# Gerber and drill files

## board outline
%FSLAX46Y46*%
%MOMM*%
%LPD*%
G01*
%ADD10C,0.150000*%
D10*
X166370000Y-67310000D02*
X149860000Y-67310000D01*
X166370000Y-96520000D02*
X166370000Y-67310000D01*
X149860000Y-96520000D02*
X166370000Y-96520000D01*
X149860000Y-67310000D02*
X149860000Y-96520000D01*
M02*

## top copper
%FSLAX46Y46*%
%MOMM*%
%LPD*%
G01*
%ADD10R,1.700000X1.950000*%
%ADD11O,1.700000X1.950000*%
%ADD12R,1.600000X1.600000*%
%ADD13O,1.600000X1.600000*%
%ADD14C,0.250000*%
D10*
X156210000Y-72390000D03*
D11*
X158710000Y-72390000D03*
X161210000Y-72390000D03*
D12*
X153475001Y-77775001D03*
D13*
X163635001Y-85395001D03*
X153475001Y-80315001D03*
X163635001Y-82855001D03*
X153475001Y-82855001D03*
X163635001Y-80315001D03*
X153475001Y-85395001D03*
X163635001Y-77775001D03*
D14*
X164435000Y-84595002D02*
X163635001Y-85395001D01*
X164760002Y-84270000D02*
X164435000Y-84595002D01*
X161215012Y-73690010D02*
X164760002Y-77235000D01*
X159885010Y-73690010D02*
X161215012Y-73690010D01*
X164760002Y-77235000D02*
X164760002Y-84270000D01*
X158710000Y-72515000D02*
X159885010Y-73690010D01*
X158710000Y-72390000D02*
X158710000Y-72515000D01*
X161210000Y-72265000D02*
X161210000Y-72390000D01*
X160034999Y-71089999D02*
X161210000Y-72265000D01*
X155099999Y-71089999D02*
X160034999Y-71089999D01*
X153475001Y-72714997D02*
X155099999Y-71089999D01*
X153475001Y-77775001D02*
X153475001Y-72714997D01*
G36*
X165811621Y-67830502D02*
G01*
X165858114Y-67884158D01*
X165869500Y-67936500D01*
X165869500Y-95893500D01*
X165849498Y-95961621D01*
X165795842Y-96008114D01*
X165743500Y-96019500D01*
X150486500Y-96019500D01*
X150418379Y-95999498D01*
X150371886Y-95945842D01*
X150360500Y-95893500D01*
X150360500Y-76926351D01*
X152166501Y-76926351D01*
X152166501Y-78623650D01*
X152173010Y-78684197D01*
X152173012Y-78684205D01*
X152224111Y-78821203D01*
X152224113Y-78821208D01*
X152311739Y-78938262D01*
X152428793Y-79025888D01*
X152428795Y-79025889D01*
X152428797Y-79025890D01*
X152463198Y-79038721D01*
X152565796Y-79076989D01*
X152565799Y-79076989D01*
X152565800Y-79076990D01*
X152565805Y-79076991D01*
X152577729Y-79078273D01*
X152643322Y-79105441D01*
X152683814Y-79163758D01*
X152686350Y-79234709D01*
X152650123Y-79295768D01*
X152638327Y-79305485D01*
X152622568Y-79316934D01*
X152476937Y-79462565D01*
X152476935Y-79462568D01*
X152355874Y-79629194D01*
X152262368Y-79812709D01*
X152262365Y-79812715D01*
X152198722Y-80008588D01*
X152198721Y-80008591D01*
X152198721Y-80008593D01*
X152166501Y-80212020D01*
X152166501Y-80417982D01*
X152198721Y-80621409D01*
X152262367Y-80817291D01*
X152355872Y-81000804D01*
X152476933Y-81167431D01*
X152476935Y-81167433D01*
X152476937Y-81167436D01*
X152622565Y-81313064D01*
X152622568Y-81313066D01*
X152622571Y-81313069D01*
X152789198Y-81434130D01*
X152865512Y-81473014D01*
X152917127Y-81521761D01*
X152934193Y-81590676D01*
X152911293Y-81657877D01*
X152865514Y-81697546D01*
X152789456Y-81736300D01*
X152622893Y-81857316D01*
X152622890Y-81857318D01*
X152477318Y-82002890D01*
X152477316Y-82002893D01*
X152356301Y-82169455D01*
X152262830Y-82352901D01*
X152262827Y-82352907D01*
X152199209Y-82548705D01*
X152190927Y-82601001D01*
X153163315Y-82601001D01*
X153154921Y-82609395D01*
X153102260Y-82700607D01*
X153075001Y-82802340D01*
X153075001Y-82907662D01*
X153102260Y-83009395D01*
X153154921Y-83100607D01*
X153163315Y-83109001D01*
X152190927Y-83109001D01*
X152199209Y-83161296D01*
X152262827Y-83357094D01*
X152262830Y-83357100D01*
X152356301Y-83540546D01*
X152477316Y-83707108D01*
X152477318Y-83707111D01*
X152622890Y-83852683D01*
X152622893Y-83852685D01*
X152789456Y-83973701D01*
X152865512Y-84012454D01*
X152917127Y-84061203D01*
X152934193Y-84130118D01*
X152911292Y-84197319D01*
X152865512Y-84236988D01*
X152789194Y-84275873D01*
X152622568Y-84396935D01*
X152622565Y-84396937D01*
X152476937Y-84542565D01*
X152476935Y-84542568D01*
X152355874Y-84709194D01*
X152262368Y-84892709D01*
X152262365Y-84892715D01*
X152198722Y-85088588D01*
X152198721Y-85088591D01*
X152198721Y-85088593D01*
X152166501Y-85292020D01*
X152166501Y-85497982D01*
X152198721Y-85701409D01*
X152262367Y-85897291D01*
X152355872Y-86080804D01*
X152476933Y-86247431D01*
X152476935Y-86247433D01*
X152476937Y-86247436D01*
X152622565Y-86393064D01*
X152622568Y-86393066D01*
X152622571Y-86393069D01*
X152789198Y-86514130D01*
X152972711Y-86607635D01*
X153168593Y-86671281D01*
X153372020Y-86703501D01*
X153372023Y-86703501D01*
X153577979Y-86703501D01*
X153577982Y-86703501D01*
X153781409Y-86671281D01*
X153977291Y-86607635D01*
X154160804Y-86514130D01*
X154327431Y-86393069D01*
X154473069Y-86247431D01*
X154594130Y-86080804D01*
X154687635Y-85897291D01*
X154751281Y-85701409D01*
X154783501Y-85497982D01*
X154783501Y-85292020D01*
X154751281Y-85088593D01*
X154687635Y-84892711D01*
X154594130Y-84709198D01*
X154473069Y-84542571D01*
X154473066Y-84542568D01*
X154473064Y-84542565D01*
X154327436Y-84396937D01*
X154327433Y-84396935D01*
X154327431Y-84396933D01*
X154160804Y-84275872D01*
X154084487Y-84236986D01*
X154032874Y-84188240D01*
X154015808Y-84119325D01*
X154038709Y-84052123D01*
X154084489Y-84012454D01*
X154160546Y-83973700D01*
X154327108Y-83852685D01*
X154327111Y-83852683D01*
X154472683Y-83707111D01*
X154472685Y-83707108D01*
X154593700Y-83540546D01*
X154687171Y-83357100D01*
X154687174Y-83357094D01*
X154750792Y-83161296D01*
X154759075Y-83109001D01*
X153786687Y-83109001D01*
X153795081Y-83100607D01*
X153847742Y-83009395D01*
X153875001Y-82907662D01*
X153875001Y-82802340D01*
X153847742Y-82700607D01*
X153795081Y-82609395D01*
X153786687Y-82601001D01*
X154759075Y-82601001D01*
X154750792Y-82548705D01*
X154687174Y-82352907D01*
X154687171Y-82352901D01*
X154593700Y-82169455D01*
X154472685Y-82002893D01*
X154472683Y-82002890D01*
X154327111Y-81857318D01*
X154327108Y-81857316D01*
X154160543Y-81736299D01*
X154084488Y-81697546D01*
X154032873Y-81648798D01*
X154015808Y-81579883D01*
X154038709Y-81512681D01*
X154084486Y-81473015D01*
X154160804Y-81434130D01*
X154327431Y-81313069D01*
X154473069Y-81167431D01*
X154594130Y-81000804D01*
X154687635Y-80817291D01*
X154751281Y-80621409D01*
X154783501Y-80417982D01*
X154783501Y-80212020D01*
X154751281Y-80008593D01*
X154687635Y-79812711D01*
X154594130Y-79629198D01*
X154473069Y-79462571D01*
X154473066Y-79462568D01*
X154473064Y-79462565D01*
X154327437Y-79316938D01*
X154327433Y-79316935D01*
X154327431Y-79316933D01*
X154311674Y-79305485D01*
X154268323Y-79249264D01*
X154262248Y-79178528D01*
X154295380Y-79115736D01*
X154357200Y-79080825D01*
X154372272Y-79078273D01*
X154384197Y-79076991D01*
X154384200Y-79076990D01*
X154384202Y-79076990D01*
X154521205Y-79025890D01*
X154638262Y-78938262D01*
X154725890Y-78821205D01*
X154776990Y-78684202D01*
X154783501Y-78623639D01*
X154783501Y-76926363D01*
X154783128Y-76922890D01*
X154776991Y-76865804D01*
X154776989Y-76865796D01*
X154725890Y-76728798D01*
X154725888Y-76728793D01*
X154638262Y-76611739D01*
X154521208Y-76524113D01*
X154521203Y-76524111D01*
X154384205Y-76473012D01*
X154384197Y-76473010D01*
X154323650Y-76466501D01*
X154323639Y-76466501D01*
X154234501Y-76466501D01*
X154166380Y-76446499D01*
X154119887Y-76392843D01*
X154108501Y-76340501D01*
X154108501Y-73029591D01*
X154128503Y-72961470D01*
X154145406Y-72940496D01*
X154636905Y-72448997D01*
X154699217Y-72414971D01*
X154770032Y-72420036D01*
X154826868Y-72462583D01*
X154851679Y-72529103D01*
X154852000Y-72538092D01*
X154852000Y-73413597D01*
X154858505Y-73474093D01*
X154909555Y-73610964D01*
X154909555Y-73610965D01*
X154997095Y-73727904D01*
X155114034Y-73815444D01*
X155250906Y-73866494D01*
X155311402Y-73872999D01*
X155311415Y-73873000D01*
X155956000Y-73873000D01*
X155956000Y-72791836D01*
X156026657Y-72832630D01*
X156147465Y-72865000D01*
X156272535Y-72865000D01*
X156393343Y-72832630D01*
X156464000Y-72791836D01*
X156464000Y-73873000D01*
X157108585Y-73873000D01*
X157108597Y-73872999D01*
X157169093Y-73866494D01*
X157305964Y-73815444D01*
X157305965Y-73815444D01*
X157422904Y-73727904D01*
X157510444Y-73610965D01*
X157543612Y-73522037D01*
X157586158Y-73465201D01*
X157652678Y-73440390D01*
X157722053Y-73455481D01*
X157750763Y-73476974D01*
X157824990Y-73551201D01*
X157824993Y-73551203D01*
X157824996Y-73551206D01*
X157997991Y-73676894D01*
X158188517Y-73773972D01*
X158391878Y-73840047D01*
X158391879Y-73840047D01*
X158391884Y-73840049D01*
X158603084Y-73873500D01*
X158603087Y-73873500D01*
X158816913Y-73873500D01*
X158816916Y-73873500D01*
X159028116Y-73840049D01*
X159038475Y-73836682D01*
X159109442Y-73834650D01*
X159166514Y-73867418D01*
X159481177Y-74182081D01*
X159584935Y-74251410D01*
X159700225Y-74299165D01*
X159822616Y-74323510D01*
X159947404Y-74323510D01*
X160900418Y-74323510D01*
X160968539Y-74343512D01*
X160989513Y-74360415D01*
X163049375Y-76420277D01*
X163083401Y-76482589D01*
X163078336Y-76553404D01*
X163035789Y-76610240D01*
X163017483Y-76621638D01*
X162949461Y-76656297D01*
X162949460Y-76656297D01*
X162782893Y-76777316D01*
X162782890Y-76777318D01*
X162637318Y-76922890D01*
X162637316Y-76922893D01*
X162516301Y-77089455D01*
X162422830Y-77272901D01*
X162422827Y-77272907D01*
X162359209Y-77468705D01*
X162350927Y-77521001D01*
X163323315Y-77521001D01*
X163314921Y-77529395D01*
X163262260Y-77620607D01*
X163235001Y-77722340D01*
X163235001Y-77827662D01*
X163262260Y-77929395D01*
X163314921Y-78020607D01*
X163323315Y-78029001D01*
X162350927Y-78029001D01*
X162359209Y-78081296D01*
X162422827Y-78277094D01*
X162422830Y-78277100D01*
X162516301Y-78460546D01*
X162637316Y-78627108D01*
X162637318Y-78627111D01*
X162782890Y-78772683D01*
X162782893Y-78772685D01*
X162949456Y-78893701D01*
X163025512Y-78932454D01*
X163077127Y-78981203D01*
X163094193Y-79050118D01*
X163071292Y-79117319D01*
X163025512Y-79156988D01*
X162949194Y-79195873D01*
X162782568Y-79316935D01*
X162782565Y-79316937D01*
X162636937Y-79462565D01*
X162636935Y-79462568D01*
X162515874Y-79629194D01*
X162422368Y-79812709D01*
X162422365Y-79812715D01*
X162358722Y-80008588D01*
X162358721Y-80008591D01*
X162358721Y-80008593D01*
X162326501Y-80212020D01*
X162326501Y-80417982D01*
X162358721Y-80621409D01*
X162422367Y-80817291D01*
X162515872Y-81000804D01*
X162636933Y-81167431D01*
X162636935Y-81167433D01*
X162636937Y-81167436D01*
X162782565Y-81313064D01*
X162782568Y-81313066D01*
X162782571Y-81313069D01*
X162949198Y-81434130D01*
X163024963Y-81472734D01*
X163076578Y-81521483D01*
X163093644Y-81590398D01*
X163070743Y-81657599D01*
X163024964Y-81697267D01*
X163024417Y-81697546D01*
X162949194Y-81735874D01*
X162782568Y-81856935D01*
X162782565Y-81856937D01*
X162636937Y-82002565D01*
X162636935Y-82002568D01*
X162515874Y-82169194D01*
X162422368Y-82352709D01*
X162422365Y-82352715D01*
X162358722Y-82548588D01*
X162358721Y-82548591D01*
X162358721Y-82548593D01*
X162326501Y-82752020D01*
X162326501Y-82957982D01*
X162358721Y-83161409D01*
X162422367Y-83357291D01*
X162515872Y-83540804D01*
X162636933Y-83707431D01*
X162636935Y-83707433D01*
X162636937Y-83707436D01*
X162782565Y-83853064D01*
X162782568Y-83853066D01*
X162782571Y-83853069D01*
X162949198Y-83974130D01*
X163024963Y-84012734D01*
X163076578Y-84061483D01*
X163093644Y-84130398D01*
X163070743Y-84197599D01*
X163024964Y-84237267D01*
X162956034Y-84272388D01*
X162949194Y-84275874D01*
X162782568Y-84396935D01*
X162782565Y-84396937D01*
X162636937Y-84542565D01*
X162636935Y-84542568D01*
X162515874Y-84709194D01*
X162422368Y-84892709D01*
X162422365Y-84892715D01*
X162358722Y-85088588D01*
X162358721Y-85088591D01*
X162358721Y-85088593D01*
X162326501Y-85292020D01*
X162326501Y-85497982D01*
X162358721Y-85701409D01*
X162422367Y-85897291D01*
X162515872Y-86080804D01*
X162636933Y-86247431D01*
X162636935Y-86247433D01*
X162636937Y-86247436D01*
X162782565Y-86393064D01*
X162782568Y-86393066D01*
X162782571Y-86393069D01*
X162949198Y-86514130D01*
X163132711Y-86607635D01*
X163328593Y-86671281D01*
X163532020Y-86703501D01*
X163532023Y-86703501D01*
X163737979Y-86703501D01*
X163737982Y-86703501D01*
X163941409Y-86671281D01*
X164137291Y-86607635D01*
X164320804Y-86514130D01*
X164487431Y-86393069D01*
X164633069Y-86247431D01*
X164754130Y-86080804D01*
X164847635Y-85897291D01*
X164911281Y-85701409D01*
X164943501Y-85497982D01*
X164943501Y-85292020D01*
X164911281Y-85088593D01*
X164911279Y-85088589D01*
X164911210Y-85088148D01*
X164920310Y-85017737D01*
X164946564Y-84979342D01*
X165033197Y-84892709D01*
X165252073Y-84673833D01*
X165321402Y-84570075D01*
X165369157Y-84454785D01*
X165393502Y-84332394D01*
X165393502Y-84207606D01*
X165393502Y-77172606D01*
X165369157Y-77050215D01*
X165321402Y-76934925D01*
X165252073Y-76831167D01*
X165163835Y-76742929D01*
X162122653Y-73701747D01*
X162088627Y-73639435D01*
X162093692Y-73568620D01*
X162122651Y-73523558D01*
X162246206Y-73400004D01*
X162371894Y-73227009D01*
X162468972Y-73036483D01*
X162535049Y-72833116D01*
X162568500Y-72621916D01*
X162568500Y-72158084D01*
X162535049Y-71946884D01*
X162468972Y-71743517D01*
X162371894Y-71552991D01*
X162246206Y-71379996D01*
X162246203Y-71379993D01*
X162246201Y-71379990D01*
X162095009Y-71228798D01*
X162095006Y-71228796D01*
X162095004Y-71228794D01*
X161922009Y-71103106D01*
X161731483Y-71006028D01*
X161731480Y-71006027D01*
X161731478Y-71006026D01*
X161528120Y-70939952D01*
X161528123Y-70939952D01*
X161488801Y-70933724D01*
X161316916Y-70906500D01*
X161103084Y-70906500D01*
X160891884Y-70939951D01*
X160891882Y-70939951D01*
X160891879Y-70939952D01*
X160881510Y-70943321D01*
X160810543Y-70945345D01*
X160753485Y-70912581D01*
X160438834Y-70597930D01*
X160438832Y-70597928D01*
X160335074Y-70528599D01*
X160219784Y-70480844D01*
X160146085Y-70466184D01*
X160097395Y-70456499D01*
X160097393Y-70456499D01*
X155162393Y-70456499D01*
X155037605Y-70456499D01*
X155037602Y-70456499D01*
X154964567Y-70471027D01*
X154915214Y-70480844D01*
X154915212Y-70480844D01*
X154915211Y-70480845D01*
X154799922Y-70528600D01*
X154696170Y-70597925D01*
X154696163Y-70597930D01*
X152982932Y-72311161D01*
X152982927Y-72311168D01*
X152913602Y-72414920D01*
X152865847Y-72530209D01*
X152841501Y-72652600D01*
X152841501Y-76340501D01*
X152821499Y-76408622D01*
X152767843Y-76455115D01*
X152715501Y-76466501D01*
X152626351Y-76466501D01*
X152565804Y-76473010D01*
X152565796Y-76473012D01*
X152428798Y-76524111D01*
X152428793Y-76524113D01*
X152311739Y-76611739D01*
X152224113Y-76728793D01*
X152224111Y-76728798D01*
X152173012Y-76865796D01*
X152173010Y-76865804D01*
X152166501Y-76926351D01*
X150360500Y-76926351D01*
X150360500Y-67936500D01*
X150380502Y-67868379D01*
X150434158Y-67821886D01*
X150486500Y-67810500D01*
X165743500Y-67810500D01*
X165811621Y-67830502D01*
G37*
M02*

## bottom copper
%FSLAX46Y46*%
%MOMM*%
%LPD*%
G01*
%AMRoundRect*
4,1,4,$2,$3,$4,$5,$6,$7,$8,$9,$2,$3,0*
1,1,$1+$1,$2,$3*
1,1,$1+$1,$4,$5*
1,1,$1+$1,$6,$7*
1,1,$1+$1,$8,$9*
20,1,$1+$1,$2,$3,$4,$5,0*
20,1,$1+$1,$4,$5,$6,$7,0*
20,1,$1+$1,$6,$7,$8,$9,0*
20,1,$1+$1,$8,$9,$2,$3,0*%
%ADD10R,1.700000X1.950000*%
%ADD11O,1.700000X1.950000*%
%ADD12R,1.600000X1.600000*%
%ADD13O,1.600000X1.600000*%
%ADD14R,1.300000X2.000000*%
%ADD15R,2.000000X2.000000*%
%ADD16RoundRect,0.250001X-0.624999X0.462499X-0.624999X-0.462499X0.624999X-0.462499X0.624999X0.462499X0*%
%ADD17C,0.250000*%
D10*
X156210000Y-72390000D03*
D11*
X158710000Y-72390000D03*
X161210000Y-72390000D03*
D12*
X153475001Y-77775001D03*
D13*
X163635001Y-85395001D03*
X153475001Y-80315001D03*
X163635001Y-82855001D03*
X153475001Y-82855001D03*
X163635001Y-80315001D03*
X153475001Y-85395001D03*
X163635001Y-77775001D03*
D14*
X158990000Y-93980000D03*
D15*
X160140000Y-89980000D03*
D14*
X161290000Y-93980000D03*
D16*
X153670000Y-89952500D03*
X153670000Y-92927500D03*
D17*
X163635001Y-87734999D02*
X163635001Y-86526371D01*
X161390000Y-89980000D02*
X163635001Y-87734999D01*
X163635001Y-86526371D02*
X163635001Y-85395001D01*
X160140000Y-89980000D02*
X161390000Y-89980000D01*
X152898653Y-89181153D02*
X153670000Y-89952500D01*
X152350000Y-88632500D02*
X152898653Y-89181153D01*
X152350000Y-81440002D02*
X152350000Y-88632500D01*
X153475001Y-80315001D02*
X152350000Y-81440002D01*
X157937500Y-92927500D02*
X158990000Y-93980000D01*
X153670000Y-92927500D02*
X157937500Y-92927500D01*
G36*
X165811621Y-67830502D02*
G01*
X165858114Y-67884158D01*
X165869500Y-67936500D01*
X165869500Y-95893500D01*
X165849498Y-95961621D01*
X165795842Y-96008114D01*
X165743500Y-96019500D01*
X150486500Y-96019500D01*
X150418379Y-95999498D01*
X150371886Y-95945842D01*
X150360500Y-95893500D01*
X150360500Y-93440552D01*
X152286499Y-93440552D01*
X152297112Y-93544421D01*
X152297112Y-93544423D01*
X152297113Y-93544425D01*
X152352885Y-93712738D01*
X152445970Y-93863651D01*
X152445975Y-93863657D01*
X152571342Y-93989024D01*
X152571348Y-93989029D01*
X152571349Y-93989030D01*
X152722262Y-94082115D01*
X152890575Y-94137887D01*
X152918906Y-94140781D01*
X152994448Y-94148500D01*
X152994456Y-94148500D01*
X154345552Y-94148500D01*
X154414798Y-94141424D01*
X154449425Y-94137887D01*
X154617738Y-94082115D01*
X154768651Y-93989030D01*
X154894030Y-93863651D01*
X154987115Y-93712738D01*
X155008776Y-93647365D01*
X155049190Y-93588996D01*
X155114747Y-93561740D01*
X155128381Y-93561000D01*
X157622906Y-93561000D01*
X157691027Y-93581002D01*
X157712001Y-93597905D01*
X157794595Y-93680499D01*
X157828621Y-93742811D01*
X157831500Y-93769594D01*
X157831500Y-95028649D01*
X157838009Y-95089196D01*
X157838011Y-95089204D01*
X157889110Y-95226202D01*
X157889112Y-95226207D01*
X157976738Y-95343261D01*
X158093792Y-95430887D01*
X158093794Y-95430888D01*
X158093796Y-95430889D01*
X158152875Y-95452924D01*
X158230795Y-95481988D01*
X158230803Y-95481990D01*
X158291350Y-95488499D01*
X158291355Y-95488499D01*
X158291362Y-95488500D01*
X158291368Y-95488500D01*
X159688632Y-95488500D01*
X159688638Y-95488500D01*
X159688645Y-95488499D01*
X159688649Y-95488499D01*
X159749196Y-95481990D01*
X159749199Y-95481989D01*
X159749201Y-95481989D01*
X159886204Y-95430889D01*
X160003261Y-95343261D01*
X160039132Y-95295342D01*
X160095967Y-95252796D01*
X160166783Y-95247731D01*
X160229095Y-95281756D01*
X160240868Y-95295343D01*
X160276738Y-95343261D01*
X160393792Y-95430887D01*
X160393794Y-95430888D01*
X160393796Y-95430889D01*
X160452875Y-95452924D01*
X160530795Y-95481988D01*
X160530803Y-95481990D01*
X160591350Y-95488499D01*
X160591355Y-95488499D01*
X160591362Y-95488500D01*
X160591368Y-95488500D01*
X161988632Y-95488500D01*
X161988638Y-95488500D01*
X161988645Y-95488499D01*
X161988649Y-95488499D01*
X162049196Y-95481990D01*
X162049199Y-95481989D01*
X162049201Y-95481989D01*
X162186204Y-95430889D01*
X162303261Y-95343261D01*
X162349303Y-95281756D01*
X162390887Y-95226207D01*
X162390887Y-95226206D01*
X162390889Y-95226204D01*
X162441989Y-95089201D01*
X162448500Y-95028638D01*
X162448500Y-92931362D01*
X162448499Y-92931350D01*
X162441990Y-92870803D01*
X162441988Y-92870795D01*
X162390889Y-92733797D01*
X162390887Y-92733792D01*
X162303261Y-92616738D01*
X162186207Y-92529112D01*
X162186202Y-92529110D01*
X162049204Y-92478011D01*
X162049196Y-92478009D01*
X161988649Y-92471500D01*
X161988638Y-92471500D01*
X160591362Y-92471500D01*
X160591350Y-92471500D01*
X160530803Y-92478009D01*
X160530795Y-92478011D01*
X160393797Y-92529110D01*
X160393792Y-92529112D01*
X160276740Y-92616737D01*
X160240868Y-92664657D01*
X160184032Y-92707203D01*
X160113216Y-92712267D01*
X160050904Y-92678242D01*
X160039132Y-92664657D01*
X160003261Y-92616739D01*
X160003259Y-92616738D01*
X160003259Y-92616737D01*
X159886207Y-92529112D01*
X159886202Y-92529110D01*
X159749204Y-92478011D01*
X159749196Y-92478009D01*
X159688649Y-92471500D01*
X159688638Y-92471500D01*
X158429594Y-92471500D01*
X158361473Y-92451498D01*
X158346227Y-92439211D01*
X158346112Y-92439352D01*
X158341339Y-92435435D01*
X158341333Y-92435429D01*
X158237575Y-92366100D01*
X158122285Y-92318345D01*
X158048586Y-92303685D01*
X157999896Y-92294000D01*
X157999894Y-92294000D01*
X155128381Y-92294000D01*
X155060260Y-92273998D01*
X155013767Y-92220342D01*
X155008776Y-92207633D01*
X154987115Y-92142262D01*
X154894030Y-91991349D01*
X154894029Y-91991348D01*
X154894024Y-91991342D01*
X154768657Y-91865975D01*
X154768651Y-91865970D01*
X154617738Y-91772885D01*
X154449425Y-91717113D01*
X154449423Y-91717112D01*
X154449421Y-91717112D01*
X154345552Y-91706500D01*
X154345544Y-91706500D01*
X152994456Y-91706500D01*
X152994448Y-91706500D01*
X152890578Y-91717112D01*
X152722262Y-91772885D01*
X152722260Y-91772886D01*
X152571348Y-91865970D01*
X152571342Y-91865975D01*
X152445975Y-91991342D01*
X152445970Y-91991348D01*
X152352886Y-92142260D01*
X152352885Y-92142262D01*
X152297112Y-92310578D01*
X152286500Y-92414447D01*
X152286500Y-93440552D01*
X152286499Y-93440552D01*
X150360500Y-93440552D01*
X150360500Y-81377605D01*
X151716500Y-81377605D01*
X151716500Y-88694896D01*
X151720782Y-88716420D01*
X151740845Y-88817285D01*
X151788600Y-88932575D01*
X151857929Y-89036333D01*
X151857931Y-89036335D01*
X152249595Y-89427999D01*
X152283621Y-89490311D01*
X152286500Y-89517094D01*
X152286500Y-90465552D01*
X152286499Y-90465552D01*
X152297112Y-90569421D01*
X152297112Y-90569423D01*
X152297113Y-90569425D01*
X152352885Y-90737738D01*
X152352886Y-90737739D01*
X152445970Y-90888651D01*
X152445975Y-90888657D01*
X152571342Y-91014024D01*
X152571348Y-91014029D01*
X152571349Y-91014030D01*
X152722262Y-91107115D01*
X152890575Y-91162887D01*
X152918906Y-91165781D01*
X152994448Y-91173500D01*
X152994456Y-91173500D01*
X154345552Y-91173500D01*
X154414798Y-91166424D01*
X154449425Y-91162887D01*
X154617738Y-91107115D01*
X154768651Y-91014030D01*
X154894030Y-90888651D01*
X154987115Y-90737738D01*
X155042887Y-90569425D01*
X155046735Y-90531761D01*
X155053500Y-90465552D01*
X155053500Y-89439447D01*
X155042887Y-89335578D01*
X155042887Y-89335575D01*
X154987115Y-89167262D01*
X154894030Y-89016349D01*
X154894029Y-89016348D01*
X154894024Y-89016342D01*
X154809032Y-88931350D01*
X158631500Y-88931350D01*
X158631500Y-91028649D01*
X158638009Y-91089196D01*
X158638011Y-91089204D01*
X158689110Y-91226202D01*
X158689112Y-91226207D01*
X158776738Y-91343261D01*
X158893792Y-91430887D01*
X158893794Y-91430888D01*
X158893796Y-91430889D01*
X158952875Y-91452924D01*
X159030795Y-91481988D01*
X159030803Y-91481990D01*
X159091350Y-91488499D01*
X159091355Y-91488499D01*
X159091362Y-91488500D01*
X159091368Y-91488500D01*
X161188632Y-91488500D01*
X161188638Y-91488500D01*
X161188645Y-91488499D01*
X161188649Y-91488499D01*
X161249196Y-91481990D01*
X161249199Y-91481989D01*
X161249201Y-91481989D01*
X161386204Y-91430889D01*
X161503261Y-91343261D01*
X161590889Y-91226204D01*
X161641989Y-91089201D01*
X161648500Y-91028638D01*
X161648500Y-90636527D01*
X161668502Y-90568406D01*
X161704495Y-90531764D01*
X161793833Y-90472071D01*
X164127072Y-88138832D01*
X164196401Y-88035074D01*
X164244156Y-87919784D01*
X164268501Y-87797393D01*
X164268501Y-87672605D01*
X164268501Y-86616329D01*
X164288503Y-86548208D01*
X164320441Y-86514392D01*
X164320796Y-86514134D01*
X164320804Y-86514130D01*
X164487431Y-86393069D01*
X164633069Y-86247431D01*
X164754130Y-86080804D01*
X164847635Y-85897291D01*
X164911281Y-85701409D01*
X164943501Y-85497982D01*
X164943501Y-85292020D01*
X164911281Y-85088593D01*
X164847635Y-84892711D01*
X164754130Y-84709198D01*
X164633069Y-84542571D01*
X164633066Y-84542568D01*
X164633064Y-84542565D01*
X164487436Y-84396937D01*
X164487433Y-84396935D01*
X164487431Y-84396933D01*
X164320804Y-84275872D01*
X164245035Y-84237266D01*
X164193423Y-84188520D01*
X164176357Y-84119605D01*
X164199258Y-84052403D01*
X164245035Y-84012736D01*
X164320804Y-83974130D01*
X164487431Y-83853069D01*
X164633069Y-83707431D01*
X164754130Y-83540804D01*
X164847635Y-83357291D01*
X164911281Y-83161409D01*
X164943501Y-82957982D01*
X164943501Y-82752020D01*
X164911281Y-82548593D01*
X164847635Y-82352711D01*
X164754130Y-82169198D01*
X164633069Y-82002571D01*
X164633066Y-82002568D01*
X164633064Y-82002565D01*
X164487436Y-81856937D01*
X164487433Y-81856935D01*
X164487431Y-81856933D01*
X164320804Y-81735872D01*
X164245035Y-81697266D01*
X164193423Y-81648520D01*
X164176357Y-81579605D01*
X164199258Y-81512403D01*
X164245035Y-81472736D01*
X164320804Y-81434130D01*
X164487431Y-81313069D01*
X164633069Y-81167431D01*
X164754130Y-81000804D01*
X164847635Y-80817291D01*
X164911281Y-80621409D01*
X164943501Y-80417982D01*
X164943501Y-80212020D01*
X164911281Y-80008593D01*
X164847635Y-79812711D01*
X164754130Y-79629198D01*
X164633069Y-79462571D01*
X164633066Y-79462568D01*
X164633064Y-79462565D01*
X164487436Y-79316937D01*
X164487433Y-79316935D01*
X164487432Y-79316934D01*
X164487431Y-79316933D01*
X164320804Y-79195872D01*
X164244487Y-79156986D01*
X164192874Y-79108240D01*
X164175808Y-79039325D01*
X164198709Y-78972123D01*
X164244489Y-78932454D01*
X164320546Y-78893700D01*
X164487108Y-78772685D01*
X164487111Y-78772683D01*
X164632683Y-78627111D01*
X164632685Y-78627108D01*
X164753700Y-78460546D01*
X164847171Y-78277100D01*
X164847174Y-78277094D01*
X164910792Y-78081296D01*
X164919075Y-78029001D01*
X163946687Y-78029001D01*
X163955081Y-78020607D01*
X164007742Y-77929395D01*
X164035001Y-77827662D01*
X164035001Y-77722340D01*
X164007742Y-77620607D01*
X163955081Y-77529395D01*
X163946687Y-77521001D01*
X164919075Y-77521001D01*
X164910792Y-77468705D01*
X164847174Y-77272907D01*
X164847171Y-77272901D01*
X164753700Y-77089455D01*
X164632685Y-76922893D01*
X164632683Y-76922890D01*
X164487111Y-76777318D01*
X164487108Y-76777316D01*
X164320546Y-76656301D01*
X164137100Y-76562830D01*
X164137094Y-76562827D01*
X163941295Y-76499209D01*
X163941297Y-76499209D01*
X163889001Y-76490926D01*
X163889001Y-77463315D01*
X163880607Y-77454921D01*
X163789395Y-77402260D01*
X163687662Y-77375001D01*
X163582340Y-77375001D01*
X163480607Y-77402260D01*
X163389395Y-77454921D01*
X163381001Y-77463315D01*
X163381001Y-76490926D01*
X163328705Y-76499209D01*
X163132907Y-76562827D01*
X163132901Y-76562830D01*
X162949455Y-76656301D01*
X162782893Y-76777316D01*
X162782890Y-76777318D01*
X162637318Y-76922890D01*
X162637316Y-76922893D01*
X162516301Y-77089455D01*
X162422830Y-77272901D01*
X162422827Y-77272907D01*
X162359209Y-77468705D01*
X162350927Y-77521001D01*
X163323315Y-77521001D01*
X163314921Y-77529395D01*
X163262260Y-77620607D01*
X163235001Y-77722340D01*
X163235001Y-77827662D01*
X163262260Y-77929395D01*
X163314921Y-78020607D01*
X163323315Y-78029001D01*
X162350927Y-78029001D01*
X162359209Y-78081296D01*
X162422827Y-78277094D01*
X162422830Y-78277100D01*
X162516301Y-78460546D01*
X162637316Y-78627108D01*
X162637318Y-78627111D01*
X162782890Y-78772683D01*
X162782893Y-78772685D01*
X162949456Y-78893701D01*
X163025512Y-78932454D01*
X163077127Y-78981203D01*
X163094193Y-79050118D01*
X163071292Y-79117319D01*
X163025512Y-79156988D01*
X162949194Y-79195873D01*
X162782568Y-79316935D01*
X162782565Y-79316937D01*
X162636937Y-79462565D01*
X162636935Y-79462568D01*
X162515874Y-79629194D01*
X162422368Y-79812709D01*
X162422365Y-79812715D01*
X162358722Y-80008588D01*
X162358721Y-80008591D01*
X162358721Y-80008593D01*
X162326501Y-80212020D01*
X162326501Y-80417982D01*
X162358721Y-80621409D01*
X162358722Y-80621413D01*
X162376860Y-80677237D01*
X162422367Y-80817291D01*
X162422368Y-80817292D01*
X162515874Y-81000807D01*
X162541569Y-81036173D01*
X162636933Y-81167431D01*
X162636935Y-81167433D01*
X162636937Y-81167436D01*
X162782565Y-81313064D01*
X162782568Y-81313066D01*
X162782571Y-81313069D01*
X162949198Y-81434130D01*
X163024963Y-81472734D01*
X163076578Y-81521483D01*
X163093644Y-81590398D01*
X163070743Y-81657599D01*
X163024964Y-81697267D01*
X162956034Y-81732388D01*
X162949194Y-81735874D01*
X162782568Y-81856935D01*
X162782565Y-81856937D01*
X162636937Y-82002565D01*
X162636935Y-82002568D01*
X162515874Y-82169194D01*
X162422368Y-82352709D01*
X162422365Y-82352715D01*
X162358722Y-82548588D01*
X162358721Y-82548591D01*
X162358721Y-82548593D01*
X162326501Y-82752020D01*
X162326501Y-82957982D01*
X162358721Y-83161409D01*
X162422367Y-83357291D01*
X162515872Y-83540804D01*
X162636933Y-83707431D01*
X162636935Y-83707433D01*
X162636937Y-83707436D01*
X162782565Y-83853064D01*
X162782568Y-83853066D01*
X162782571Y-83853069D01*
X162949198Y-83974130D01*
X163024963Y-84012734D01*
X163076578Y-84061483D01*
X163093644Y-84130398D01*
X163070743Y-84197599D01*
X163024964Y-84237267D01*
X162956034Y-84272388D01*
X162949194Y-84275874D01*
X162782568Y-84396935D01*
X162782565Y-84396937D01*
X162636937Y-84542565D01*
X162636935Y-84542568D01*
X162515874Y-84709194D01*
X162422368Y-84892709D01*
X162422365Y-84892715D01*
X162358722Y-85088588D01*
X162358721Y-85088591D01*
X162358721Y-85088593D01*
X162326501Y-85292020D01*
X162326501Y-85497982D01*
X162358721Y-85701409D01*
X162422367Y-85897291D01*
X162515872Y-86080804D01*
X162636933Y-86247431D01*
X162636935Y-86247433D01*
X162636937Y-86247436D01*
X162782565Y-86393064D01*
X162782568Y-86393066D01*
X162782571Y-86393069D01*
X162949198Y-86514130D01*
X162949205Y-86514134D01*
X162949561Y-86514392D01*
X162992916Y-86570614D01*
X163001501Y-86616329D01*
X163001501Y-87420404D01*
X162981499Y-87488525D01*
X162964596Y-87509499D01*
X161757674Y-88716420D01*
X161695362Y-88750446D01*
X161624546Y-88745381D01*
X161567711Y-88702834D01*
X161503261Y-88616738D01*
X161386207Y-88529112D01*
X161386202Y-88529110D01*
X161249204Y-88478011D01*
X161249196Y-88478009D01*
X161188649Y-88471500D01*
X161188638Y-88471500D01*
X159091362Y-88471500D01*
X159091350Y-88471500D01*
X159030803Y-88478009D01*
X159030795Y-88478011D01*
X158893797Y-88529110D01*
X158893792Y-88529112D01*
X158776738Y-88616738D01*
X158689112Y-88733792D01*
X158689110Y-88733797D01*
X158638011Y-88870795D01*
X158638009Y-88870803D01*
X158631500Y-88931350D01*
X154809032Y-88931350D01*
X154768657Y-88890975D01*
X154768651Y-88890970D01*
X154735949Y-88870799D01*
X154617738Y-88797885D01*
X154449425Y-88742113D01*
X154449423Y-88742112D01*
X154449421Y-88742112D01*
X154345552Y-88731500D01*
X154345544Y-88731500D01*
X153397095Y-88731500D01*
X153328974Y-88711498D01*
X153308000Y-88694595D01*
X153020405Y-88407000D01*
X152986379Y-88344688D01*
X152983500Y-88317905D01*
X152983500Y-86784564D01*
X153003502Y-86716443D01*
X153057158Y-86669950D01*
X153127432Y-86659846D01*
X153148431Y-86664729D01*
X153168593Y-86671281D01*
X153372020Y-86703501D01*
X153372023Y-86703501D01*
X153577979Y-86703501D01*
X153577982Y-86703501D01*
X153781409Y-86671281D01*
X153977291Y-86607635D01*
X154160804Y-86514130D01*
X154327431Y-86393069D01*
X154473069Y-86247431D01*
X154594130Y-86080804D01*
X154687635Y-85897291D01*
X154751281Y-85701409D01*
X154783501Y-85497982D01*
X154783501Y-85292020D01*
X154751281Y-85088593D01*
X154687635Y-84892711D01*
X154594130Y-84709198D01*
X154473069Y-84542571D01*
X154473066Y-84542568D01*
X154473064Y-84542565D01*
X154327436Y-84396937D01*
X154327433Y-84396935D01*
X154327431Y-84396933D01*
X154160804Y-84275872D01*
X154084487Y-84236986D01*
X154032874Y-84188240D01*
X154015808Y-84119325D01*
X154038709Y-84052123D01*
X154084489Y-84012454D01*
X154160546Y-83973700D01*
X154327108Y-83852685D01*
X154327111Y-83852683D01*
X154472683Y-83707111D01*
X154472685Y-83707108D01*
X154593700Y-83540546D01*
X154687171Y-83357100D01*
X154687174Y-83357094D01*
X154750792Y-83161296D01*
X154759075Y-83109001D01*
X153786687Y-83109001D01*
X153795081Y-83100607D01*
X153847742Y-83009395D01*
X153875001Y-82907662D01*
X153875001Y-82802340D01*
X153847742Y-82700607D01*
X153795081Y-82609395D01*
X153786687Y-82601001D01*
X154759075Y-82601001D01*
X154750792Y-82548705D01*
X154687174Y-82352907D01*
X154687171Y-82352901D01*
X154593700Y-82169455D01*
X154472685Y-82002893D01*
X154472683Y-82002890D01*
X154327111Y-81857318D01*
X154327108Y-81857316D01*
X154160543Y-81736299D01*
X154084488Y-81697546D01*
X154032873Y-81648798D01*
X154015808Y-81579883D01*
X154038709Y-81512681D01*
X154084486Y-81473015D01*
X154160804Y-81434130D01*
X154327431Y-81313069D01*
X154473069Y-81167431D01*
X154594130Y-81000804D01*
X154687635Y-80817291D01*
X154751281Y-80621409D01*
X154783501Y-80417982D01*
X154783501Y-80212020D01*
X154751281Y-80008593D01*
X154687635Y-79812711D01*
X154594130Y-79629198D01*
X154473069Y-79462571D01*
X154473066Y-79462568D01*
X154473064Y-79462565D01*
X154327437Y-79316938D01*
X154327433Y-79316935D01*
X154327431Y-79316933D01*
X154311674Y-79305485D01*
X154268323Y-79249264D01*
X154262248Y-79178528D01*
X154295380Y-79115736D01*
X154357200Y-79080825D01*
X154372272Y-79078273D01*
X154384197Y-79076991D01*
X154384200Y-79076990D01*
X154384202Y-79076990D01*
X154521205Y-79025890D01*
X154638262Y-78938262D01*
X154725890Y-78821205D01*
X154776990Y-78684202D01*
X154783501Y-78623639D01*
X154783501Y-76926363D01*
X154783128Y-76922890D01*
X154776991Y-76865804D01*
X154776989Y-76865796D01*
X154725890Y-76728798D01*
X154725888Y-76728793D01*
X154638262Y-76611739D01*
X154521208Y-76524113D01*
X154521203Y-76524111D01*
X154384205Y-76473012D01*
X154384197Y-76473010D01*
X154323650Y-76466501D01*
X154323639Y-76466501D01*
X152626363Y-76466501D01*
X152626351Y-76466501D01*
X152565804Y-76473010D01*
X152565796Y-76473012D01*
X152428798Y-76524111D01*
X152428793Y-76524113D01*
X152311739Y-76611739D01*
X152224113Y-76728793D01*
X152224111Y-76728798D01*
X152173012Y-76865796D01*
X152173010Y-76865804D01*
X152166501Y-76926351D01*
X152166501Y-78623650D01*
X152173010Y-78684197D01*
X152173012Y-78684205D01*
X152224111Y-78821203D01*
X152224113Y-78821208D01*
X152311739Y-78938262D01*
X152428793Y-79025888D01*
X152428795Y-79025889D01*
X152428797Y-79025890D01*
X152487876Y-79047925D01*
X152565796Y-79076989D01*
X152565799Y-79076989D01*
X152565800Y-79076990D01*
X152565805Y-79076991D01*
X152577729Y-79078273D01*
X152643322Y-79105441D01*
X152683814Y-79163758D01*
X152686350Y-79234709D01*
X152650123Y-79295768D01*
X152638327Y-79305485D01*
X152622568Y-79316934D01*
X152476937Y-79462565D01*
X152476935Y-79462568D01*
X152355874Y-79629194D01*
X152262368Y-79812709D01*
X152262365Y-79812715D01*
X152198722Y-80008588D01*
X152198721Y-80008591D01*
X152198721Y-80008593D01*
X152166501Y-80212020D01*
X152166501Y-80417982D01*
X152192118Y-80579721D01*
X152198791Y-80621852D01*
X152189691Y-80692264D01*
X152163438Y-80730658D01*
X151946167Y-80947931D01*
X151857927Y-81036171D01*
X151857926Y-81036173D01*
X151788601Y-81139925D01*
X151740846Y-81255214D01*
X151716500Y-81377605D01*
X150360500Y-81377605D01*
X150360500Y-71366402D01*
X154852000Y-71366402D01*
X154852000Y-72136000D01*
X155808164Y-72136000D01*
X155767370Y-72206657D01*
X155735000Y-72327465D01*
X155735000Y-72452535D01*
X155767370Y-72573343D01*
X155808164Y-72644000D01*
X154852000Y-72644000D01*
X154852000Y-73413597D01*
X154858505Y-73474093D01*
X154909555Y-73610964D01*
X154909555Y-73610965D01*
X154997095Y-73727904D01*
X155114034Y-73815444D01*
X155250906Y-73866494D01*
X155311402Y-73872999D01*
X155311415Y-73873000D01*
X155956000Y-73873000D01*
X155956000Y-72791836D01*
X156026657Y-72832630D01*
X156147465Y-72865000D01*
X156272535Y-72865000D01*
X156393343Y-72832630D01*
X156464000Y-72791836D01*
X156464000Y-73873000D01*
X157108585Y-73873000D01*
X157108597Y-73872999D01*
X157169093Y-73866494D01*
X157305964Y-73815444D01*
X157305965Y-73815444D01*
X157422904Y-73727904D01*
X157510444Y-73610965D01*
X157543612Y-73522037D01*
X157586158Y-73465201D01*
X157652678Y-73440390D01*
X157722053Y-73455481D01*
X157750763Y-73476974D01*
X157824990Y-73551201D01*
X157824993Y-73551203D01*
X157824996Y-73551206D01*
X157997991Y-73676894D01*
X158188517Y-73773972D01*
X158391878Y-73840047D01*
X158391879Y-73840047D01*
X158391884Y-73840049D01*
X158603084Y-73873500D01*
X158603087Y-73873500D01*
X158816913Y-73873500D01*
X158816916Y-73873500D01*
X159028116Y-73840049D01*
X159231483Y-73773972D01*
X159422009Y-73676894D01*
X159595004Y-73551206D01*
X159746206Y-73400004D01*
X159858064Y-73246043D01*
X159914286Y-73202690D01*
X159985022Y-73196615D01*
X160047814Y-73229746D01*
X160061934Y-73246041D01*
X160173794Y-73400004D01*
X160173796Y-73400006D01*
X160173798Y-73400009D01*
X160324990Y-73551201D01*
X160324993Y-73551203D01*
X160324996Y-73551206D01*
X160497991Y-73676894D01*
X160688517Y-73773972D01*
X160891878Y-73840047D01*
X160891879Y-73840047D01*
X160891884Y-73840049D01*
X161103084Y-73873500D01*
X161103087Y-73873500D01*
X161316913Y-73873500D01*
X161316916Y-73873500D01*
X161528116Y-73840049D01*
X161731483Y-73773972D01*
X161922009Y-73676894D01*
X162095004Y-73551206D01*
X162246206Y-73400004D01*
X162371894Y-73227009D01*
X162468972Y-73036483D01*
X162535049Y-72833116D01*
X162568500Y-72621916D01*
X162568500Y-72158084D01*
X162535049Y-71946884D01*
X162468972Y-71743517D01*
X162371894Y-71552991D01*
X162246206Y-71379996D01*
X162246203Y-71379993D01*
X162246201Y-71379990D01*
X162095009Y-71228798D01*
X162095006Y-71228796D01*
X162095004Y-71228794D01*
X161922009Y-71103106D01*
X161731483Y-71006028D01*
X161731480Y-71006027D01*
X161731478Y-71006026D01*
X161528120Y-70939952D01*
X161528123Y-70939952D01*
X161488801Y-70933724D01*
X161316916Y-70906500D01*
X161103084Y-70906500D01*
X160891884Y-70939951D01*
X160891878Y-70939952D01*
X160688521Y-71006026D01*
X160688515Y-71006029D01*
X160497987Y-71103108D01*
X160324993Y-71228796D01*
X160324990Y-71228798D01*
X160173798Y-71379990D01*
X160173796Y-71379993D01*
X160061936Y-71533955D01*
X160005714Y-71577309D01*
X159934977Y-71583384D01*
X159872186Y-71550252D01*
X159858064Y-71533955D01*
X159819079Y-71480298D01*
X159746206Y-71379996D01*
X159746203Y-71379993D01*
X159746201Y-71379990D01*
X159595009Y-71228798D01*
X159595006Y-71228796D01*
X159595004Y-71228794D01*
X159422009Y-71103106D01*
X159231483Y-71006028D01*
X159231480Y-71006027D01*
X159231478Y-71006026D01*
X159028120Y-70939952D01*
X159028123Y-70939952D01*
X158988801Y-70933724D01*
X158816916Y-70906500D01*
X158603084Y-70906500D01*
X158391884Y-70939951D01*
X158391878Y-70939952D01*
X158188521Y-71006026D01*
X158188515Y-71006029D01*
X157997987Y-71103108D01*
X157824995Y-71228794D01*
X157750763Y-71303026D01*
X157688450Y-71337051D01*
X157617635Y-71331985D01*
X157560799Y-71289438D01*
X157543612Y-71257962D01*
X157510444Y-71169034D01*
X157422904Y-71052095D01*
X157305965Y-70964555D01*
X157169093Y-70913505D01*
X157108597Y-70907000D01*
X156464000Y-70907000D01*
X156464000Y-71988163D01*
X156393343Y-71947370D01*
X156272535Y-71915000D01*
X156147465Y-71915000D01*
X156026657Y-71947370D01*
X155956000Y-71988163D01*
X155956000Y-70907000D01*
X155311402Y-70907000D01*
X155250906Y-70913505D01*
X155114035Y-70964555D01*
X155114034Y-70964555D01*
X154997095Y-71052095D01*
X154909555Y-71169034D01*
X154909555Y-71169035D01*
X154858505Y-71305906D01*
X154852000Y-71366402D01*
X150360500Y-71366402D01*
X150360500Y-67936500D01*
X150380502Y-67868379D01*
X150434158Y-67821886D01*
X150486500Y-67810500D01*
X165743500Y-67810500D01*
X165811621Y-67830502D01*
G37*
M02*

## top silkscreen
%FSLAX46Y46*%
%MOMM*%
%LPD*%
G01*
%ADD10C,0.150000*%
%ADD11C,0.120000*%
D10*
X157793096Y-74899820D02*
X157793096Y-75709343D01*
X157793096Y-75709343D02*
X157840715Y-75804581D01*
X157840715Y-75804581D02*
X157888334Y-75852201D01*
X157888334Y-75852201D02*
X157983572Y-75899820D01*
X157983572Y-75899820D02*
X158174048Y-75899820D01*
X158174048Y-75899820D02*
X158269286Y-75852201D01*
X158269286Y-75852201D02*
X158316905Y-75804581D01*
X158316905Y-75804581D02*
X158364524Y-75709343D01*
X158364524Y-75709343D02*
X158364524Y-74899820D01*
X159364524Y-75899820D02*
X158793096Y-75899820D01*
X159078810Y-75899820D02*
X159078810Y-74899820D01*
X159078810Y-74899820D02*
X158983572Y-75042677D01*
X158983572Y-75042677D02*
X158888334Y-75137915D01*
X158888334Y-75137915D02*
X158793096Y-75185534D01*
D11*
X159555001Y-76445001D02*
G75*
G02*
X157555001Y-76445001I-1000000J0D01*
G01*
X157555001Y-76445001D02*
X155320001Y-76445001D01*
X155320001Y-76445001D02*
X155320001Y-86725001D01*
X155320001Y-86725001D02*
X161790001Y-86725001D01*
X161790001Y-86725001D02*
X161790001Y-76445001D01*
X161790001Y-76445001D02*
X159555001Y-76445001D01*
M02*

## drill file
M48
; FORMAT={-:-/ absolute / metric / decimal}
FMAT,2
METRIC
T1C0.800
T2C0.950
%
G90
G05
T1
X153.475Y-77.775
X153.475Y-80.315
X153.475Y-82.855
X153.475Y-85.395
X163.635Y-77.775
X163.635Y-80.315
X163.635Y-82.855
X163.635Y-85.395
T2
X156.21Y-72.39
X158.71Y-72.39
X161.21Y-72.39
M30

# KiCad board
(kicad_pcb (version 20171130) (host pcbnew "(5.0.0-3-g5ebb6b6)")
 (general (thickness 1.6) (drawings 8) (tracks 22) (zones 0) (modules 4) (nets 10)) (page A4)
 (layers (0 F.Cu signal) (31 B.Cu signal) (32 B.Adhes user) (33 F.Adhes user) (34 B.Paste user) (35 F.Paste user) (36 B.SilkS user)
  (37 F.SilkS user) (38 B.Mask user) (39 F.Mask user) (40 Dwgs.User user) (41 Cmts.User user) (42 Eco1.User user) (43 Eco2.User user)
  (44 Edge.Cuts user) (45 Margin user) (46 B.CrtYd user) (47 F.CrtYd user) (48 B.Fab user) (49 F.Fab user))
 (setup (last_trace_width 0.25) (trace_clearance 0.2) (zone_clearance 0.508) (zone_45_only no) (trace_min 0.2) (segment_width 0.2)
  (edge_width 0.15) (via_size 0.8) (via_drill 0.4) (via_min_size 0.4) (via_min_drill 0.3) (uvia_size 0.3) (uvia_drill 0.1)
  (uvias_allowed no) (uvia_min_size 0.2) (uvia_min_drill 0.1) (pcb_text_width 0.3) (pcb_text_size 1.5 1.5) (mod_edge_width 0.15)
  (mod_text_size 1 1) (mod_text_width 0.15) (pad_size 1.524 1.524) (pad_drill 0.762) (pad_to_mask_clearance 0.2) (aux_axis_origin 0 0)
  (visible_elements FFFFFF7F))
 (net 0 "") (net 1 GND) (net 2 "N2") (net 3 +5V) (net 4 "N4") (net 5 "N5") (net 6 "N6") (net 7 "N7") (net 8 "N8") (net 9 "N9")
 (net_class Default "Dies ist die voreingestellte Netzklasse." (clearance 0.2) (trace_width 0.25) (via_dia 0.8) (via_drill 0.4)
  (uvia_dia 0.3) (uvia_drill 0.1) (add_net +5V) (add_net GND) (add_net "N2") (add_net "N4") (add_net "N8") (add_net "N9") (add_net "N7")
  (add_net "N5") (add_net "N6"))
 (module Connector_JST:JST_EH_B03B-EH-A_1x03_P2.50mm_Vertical (layer B.Cu) (at 156.21 72.39)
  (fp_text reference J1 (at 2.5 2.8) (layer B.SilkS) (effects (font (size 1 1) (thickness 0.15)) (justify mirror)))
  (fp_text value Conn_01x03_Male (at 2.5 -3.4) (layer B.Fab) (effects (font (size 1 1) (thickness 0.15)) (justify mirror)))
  (pad 1 thru_hole rect (at 0 0) (size 1.7 1.95) (drill 0.95) (layers *.Cu *.Mask) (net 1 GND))
  (pad 2 thru_hole oval (at 2.5 0) (size 1.7 1.95) (drill 0.95) (layers *.Cu *.Mask) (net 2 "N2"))
  (pad 3 thru_hole oval (at 5 0) (size 1.7 1.95) (drill 0.95) (layers *.Cu *.Mask) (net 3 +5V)))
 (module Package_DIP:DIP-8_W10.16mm (layer F.Cu) (at 153.475001 77.775001)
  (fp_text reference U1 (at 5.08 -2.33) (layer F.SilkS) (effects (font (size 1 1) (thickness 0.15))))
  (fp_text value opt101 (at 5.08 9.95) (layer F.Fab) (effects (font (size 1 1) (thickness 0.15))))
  (fp_arc (start 5.08 -1.33) (end 4.08 -1.33) (angle -180) (layer F.SilkS) (width 0.12))
  (fp_line (start 4.08 -1.33) (end 1.845 -1.33) (layer F.SilkS) (width 0.12))
  (fp_line (start 1.845 -1.33) (end 1.845 8.95) (layer F.SilkS) (width 0.12))
  (fp_line (start 1.845 8.95) (end 8.315 8.95) (layer F.SilkS) (width 0.12))
  (fp_line (start 8.315 8.95) (end 8.315 -1.33) (layer F.SilkS) (width 0.12))
  (fp_line (start 8.315 -1.33) (end 6.08 -1.33) (layer F.SilkS) (width 0.12))
  (pad 1 thru_hole rect (at 0 0) (size 1.6 1.6) (drill 0.8) (layers *.Cu *.Mask) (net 3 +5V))
  (pad 5 thru_hole oval (at 10.16 7.62) (size 1.6 1.6) (drill 0.8) (layers *.Cu *.Mask) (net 2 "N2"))
  (pad 2 thru_hole oval (at 0 2.54) (size 1.6 1.6) (drill 0.8) (layers *.Cu *.Mask) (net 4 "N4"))
  (pad 6 thru_hole oval (at 10.16 5.08) (size 1.6 1.6) (drill 0.8) (layers *.Cu *.Mask) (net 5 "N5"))
  (pad 3 thru_hole oval (at 0 5.08) (size 1.6 1.6) (drill 0.8) (layers *.Cu *.Mask) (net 1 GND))
  (pad 7 thru_hole oval (at 10.16 2.54) (size 1.6 1.6) (drill 0.8) (layers *.Cu *.Mask) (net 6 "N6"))
  (pad 4 thru_hole oval (at 0 7.62) (size 1.6 1.6) (drill 0.8) (layers *.Cu *.Mask) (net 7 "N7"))
  (pad 8 thru_hole oval (at 10.16 0) (size 1.6 1.6) (drill 0.8) (layers *.Cu *.Mask) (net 1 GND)))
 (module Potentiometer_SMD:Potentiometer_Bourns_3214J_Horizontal (layer B.Cu) (at 160.14 91.98 270)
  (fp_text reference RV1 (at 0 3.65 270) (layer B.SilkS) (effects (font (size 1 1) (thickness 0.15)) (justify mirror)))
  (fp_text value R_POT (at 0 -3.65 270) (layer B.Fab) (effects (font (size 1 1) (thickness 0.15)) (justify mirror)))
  (pad 1 smd rect (at 2 1.15 270) (size 2 1.3) (layers B.Cu B.Paste B.Mask) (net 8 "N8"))
  (pad 2 smd rect (at -2 0 270) (size 2 2) (layers B.Cu B.Paste B.Mask) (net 2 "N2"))
  (pad 3 smd rect (at 2 -1.15 270) (size 2 1.3) (layers B.Cu B.Paste B.Mask) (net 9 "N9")))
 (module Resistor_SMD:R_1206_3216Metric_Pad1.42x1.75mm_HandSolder (layer B.Cu) (at 153.67 91.44 270)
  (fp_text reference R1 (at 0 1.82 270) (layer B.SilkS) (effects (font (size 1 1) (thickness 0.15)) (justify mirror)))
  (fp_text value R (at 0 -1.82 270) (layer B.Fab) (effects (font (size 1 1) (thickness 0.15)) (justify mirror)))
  (pad 1 smd roundrect (at -1.4875 0 270) (size 1.425 1.75) (layers B.Cu B.Paste B.Mask) (roundrect_rratio 0.175439) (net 4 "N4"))
  (pad 2 smd roundrect (at 1.4875 0 270) (size 1.425 1.75) (layers B.Cu B.Paste B.Mask) (roundrect_rratio 0.175439) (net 8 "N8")))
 (gr_line (start 166.37 67.31) (end 149.86 67.31) (layer Edge.Cuts) (width 0.15))
 (gr_line (start 166.37 96.52) (end 166.37 67.31) (layer Edge.Cuts) (width 0.15))
 (gr_line (start 149.86 96.52) (end 166.37 96.52) (layer Edge.Cuts) (width 0.15))
 (gr_line (start 149.86 67.31) (end 149.86 96.52) (layer Edge.Cuts) (width 0.15))
 (segment (start 164.435 84.595002) (end 163.635001 85.395001) (width 0.25) (layer F.Cu) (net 2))
 (segment (start 164.760002 84.27) (end 164.435 84.595002) (width 0.25) (layer F.Cu) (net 2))
 (segment (start 161.215012 73.69001) (end 164.760002 77.235) (width 0.25) (layer F.Cu) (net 2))
 (segment (start 159.88501 73.69001) (end 161.215012 73.69001) (width 0.25) (layer F.Cu) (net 2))
 (segment (start 164.760002 77.235) (end 164.760002 84.27) (width 0.25) (layer F.Cu) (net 2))
 (segment (start 158.71 72.515) (end 159.88501 73.69001) (width 0.25) (layer F.Cu) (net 2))
 (segment (start 158.71 72.39) (end 158.71 72.515) (width 0.25) (layer F.Cu) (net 2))
 (segment (start 163.635001 87.734999) (end 163.635001 86.526371) (width 0.25) (layer B.Cu) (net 2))
 (segment (start 161.39 89.98) (end 163.635001 87.734999) (width 0.25) (layer B.Cu) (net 2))
 (segment (start 163.635001 86.526371) (end 163.635001 85.395001) (width 0.25) (layer B.Cu) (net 2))
 (segment (start 160.14 89.98) (end 161.39 89.98) (width 0.25) (layer B.Cu) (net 2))
 (segment (start 161.21 72.265) (end 161.21 72.39) (width 0.25) (layer F.Cu) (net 3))
 (segment (start 160.034999 71.089999) (end 161.21 72.265) (width 0.25) (layer F.Cu) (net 3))
 (segment (start 155.099999 71.089999) (end 160.034999 71.089999) (width 0.25) (layer F.Cu) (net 3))
 (segment (start 153.475001 72.714997) (end 155.099999 71.089999) (width 0.25) (layer F.Cu) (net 3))
 (segment (start 153.475001 77.775001) (end 153.475001 72.714997) (width 0.25) (layer F.Cu) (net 3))
 (segment (start 152.898653 89.181153) (end 153.67 89.9525) (width 0.25) (layer B.Cu) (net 4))
 (segment (start 152.35 88.6325) (end 152.898653 89.181153) (width 0.25) (layer B.Cu) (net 4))
 (segment (start 152.35 81.440002) (end 152.35 88.6325) (width 0.25) (layer B.Cu) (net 4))
 (segment (start 153.475001 80.315001) (end 152.35 81.440002) (width 0.25) (layer B.Cu) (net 4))
 (segment (start 157.9375 92.9275) (end 158.99 93.98) (width 0.25) (layer B.Cu) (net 8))
 (segment (start 153.67 92.9275) (end 157.9375 92.9275) (width 0.25) (layer B.Cu) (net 8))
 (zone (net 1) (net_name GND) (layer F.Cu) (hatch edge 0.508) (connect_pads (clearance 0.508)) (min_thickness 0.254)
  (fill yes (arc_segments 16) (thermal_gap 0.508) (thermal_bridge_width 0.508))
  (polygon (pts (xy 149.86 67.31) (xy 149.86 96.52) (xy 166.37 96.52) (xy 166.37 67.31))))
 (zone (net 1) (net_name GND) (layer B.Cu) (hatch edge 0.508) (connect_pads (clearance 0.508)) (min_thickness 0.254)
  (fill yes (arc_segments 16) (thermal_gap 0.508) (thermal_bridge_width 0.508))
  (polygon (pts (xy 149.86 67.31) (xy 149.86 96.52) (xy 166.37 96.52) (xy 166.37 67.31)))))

